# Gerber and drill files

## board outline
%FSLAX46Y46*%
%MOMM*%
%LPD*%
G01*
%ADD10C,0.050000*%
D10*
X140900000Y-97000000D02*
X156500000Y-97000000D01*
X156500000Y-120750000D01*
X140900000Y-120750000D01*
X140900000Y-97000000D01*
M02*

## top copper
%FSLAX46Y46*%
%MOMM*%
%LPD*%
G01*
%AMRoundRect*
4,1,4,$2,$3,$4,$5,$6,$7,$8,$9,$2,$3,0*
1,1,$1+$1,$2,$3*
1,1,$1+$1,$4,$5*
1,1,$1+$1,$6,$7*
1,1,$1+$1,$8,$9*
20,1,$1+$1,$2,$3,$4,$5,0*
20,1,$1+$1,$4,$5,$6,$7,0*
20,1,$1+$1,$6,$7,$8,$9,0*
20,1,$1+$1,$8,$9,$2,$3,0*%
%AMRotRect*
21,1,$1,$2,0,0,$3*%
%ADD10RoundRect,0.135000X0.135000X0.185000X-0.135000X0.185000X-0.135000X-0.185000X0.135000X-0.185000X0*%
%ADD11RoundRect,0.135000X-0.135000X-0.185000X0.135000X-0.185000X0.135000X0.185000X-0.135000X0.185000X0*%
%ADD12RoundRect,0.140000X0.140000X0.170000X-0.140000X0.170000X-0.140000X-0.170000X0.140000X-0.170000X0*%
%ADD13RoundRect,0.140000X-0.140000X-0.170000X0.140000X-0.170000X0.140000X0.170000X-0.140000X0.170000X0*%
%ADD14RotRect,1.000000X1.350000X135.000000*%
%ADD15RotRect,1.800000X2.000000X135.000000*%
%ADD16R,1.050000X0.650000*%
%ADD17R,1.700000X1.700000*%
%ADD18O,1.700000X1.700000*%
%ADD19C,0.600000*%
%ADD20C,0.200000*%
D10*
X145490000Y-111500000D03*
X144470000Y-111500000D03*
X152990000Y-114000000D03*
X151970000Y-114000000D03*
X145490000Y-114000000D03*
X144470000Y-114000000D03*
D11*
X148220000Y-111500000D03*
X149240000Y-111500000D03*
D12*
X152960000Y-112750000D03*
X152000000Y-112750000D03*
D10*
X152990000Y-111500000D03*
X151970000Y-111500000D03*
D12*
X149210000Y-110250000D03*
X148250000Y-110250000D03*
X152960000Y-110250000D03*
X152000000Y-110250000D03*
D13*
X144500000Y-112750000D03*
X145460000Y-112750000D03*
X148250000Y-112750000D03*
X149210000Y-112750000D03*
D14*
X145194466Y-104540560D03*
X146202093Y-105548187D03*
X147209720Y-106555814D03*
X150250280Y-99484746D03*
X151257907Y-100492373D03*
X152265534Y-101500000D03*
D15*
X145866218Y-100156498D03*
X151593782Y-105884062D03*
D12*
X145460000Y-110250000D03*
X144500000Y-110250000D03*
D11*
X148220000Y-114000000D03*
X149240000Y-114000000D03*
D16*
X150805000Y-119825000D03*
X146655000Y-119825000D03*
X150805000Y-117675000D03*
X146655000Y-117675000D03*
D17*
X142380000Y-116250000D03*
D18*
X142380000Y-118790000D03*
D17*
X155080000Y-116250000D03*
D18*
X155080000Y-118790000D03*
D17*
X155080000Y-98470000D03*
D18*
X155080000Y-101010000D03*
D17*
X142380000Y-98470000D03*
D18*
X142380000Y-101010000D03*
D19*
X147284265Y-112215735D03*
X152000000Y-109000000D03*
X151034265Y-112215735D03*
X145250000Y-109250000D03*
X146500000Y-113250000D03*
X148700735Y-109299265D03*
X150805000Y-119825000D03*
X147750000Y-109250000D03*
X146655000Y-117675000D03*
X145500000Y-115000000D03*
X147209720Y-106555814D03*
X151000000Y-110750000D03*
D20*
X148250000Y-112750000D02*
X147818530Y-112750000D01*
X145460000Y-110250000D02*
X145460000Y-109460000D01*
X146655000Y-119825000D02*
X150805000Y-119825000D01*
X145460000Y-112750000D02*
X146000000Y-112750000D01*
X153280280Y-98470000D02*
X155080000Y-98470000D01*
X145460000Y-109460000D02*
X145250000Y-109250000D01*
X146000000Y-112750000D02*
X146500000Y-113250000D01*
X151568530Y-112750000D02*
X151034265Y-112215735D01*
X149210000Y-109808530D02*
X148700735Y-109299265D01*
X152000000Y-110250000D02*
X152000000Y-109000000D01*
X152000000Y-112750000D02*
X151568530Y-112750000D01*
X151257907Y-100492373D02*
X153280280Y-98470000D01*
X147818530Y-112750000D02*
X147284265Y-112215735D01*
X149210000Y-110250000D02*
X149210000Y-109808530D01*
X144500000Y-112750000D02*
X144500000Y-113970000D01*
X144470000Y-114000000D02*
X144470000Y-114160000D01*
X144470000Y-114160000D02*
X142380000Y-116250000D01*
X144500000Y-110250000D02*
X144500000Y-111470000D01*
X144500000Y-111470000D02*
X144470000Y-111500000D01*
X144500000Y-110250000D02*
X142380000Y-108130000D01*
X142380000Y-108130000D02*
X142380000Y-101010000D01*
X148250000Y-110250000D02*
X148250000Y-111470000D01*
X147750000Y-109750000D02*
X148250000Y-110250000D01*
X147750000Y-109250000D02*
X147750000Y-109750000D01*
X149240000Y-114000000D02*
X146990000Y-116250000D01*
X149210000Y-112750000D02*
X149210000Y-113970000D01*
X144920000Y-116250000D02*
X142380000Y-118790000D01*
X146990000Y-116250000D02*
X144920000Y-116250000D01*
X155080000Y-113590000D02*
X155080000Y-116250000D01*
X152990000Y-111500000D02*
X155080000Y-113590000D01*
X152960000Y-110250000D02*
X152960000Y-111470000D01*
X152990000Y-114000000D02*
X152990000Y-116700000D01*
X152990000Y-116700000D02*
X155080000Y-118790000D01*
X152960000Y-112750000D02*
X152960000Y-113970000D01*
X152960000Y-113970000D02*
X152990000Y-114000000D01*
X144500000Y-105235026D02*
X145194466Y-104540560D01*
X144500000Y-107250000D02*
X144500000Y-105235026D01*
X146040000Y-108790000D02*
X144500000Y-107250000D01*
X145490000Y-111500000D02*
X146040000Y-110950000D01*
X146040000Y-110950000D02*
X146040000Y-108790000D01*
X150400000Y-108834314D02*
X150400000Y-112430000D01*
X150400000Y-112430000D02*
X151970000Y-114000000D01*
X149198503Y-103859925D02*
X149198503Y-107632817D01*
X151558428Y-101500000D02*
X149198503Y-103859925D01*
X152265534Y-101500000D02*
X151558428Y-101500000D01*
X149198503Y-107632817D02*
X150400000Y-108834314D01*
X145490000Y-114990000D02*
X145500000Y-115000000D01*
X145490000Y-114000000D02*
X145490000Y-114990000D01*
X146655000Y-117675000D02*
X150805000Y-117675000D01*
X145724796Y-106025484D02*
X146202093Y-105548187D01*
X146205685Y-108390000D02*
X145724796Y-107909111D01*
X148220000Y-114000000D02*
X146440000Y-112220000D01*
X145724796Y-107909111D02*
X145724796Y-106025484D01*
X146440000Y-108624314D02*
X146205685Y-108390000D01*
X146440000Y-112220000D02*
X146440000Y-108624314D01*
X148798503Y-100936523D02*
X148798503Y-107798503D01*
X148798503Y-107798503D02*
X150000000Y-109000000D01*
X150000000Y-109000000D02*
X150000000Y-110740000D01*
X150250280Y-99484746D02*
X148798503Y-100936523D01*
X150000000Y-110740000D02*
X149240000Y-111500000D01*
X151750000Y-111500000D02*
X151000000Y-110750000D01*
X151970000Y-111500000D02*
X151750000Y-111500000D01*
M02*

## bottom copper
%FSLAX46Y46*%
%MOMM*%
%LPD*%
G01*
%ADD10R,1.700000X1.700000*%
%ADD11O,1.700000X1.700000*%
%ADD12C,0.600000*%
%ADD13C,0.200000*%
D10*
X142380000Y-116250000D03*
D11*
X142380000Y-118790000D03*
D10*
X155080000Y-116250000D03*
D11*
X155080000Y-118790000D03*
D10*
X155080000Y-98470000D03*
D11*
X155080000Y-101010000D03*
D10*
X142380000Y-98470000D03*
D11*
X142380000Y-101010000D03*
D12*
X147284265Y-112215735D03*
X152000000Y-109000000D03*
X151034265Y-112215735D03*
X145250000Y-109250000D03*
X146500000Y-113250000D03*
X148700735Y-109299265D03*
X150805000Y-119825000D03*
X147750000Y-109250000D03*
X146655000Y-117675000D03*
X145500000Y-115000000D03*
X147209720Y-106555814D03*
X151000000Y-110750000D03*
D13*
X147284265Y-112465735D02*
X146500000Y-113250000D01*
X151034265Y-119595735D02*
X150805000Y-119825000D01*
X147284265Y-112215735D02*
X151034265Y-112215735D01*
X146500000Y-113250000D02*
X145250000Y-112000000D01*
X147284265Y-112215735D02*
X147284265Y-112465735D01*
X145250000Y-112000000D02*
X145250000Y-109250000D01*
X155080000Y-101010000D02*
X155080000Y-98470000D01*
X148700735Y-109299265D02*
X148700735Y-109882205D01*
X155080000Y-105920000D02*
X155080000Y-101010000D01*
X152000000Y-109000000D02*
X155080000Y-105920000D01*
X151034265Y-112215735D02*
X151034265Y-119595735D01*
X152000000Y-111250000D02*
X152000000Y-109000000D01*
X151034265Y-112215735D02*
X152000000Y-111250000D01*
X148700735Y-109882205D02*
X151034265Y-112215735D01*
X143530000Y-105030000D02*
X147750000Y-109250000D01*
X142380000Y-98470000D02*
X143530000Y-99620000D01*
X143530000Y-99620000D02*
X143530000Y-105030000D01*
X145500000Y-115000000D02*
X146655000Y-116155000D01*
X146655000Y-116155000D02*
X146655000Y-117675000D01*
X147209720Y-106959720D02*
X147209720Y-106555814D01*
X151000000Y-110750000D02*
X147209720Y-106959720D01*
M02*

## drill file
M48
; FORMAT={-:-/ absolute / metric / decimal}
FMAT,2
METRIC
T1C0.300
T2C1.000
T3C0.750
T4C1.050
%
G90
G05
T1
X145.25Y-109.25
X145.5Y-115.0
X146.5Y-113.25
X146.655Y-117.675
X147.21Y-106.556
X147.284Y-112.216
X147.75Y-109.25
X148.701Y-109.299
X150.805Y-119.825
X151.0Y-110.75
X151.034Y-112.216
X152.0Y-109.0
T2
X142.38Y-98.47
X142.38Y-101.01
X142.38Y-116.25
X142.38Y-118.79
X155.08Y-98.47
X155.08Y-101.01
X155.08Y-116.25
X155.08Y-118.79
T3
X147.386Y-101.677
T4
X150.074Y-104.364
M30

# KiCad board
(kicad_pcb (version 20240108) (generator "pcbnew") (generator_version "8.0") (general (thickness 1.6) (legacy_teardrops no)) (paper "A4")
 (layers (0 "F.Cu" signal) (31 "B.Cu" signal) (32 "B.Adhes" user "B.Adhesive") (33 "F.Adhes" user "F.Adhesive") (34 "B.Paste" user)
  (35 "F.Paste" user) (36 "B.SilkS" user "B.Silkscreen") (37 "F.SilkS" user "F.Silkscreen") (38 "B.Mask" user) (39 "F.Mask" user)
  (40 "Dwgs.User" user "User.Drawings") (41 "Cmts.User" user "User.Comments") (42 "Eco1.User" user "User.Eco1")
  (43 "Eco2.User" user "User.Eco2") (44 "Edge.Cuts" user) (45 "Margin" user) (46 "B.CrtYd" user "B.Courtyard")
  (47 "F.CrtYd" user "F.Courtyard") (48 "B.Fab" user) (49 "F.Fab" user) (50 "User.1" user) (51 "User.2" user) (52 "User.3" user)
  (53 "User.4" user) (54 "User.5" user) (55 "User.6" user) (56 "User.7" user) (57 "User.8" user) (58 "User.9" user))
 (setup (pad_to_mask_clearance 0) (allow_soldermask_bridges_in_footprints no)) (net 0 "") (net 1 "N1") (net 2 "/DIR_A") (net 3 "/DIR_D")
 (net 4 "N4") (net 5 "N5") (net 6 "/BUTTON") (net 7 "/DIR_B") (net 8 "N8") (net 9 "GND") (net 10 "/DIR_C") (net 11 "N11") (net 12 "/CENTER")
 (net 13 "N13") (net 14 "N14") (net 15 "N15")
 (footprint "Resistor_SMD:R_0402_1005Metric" (layer "F.Cu") (at 144.98 111.5 180)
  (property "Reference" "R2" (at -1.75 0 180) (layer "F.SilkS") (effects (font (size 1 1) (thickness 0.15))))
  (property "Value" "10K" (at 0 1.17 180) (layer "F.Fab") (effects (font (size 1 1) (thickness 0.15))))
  (pad "1" smd roundrect (at -0.51 0 180) (size 0.54 0.64) (layers "F.Cu" "F.Paste" "F.Mask") (roundrect_rratio 0.25) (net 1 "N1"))
  (pad "2" smd roundrect (at 0.51 0 180) (size 0.54 0.64) (layers "F.Cu" "F.Paste" "F.Mask") (roundrect_rratio 0.25) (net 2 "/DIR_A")))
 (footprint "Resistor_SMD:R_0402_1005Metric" (layer "F.Cu") (at 152.48 114 180)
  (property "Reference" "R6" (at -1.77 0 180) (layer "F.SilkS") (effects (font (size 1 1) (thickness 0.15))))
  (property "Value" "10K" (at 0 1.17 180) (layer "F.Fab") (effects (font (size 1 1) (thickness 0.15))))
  (pad "1" smd roundrect (at -0.51 0 180) (size 0.54 0.64) (layers "F.Cu" "F.Paste" "F.Mask") (roundrect_rratio 0.25) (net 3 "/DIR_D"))
  (pad "2" smd roundrect (at 0.51 0 180) (size 0.54 0.64) (layers "F.Cu" "F.Paste" "F.Mask") (roundrect_rratio 0.25) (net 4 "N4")))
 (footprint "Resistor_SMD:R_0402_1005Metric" (layer "F.Cu") (at 144.98 114 180)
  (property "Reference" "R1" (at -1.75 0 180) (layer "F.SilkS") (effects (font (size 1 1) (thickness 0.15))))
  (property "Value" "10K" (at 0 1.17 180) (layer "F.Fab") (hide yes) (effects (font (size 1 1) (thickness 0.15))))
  (pad "1" smd roundrect (at -0.51 0 180) (size 0.54 0.64) (layers "F.Cu" "F.Paste" "F.Mask") (roundrect_rratio 0.25) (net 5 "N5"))
  (pad "2" smd roundrect (at 0.51 0 180) (size 0.54 0.64) (layers "F.Cu" "F.Paste" "F.Mask") (roundrect_rratio 0.25) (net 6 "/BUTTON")))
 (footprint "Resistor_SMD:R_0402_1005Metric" (layer "F.Cu") (at 148.73 111.5)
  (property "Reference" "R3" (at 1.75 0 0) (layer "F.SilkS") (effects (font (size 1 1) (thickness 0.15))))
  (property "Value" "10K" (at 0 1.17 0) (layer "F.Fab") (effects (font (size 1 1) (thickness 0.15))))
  (pad "1" smd roundrect (at -0.51 0) (size 0.54 0.64) (layers "F.Cu" "F.Paste" "F.Mask") (roundrect_rratio 0.25) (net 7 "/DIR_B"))
  (pad "2" smd roundrect (at 0.51 0) (size 0.54 0.64) (layers "F.Cu" "F.Paste" "F.Mask") (roundrect_rratio 0.25) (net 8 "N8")))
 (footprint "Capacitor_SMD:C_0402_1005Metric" (layer "F.Cu") (at 152.48 112.75 180)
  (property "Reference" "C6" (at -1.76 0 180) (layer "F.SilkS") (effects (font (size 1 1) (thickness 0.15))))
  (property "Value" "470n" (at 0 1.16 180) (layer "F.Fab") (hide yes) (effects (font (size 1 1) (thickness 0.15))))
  (pad "1" smd roundrect (at -0.48 0 180) (size 0.56 0.62) (layers "F.Cu" "F.Paste" "F.Mask") (roundrect_rratio 0.25) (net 3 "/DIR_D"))
  (pad "2" smd roundrect (at 0.48 0 180) (size 0.56 0.62) (layers "F.Cu" "F.Paste" "F.Mask") (roundrect_rratio 0.25) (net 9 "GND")))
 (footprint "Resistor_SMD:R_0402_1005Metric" (layer "F.Cu") (at 152.48 111.5 180)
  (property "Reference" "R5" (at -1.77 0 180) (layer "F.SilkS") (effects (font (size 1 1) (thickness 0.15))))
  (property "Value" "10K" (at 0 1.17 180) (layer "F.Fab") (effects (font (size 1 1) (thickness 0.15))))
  (pad "1" smd roundrect (at -0.51 0 180) (size 0.54 0.64) (layers "F.Cu" "F.Paste" "F.Mask") (roundrect_rratio 0.25) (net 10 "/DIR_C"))
  (pad "2" smd roundrect (at 0.51 0 180) (size 0.54 0.64) (layers "F.Cu" "F.Paste" "F.Mask") (roundrect_rratio 0.25) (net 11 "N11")))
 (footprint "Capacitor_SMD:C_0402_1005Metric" (layer "F.Cu") (at 148.73 110.25 180)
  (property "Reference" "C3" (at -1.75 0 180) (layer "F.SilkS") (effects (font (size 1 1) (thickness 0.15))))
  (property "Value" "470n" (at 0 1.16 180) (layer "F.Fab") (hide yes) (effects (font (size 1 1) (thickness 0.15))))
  (pad "1" smd roundrect (at -0.48 0 180) (size 0.56 0.62) (layers "F.Cu" "F.Paste" "F.Mask") (roundrect_rratio 0.25) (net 9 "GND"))
  (pad "2" smd roundrect (at 0.48 0 180) (size 0.56 0.62) (layers "F.Cu" "F.Paste" "F.Mask") (roundrect_rratio 0.25) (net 7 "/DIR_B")))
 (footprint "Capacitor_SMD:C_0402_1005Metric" (layer "F.Cu") (at 152.48 110.25 180)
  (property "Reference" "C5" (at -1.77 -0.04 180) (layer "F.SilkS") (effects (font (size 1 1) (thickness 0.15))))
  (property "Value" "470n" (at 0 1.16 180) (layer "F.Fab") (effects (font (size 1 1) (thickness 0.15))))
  (pad "1" smd roundrect (at -0.48 0 180) (size 0.56 0.62) (layers "F.Cu" "F.Paste" "F.Mask") (roundrect_rratio 0.25) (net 10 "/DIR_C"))
  (pad "2" smd roundrect (at 0.48 0 180) (size 0.56 0.62) (layers "F.Cu" "F.Paste" "F.Mask") (roundrect_rratio 0.25) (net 9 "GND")))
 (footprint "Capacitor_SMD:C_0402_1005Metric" (layer "F.Cu") (at 144.98 112.75)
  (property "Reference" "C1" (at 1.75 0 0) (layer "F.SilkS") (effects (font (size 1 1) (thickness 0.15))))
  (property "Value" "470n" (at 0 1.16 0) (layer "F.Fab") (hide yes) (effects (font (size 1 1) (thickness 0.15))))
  (pad "1" smd roundrect (at -0.48 0) (size 0.56 0.62) (layers "F.Cu" "F.Paste" "F.Mask") (roundrect_rratio 0.25) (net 6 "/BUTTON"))
  (pad "2" smd roundrect (at 0.48 0) (size 0.56 0.62) (layers "F.Cu" "F.Paste" "F.Mask") (roundrect_rratio 0.25) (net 9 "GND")))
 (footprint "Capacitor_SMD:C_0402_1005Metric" (layer "F.Cu") (at 148.73 112.75)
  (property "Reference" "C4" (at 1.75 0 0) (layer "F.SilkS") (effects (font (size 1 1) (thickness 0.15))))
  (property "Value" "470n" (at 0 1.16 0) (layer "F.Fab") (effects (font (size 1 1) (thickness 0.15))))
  (pad "1" smd roundrect (at -0.48 0) (size 0.56 0.62) (layers "F.Cu" "F.Paste" "F.Mask") (roundrect_rratio 0.25) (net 9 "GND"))
  (pad "2" smd roundrect (at 0.48 0) (size 0.56 0.62) (layers "F.Cu" "F.Paste" "F.Mask") (roundrect_rratio 0.25) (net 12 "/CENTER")))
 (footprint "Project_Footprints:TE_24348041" (layer "F.Cu") (at 148.73 103.02028 45)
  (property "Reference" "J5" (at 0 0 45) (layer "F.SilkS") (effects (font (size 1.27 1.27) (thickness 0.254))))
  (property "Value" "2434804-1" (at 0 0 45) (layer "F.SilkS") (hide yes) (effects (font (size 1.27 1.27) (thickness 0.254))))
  (pad "" np_thru_hole circle (at 0 -1.9 45) (size 0.75 0.75) (drill 0.75) (layers "*.Cu" "*.Mask"))
  (pad "" np_thru_hole circle (at 0 1.9 45) (size 1.05 1.05) (drill 1.05) (layers "*.Cu" "*.Mask"))
  (pad "1" smd rect (at -3.575 -1.425 135) (size 1 1.35) (layers "F.Cu" "F.Paste" "F.Mask") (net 1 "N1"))
  (pad "2" smd rect (at -3.575 0 135) (size 1 1.35) (layers "F.Cu" "F.Paste" "F.Mask") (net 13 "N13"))
  (pad "3" smd rect (at -3.575 1.425 135) (size 1 1.35) (layers "F.Cu" "F.Paste" "F.Mask") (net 11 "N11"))
  (pad "4" smd rect (at 3.575 -1.425 135) (size 1 1.35) (layers "F.Cu" "F.Paste" "F.Mask") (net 8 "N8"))
  (pad "5" smd rect (at 3.575 0 135) (size 1 1.35) (layers "F.Cu" "F.Paste" "F.Mask") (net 9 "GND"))
  (pad "6" smd rect (at 3.575 1.425 135) (size 1 1.35) (layers "F.Cu" "F.Paste" "F.Mask") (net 4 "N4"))
  (pad "MP1" smd rect (at 0 -4.049999 135) (size 1.8 2) (layers "F.Cu" "F.Paste" "F.Mask") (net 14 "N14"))
  (pad "MP2" smd rect (at 0 4.049999 135) (size 1.8 2) (layers "F.Cu" "F.Paste" "F.Mask") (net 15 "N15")))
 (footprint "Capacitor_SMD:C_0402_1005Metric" (layer "F.Cu") (at 144.98 110.25 180)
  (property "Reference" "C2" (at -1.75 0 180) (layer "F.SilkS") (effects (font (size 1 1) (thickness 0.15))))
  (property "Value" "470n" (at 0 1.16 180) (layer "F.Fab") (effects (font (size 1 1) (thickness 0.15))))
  (pad "1" smd roundrect (at -0.48 0 180) (size 0.56 0.62) (layers "F.Cu" "F.Paste" "F.Mask") (roundrect_rratio 0.25) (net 9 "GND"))
  (pad "2" smd roundrect (at 0.48 0 180) (size 0.56 0.62) (layers "F.Cu" "F.Paste" "F.Mask") (roundrect_rratio 0.25) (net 2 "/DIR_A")))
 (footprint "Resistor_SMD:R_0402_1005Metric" (layer "F.Cu") (at 148.73 114)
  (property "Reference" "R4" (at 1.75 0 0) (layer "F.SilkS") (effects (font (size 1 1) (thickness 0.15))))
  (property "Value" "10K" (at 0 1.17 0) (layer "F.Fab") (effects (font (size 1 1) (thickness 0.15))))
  (pad "1" smd roundrect (at -0.51 0) (size 0.54 0.64) (layers "F.Cu" "F.Paste" "F.Mask") (roundrect_rratio 0.25) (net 13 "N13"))
  (pad "2" smd roundrect (at 0.51 0) (size 0.54 0.64) (layers "F.Cu" "F.Paste" "F.Mask") (roundrect_rratio 0.25) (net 12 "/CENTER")))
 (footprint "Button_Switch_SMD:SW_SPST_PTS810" (layer "F.Cu") (at 148.73 118.75 180)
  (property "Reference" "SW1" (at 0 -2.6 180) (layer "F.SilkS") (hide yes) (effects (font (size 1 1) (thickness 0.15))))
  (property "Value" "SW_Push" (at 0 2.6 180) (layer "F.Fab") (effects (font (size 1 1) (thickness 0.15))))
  (pad "1" smd rect (at -2.075 -1.075 180) (size 1.05 0.65) (layers "F.Cu" "F.Paste" "F.Mask") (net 9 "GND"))
  (pad "1" smd rect (at 2.075 -1.075 180) (size 1.05 0.65) (layers "F.Cu" "F.Paste" "F.Mask") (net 9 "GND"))
  (pad "2" smd rect (at -2.075 1.075 180) (size 1.05 0.65) (layers "F.Cu" "F.Paste" "F.Mask") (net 5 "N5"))
  (pad "2" smd rect (at 2.075 1.075 180) (size 1.05 0.65) (layers "F.Cu" "F.Paste" "F.Mask") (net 5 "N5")))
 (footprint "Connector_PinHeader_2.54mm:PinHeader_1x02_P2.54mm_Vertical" (layer "B.Cu") (at 142.38 116.25 180)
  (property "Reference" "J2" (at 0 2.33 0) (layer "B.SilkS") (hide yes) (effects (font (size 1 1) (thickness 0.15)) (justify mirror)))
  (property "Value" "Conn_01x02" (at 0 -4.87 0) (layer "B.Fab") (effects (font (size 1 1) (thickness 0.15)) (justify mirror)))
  (pad "1" thru_hole rect (at 0 0 180) (size 1.7 1.7) (drill 1) (layers "*.Cu" "*.Mask") (remove_unused_layers no) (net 6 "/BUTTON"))
  (pad "2" thru_hole oval (at 0 -2.54 180) (size 1.7 1.7) (drill 1) (layers "*.Cu" "*.Mask") (remove_unused_layers no) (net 12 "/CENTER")))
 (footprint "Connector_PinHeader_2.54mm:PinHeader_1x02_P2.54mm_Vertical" (layer "B.Cu") (at 155.08 116.25 180)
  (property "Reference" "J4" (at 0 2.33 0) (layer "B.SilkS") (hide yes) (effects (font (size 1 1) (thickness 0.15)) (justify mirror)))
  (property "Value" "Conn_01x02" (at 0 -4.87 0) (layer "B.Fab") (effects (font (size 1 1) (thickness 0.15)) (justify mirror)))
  (pad "1" thru_hole rect (at 0 0 180) (size 1.7 1.7) (drill 1) (layers "*.Cu" "*.Mask") (remove_unused_layers no) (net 10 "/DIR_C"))
  (pad "2" thru_hole oval (at 0 -2.54 180) (size 1.7 1.7) (drill 1) (layers "*.Cu" "*.Mask") (remove_unused_layers no) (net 3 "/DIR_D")))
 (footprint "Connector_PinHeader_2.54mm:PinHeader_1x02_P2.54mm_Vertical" (layer "B.Cu") (at 155.08 98.47 180)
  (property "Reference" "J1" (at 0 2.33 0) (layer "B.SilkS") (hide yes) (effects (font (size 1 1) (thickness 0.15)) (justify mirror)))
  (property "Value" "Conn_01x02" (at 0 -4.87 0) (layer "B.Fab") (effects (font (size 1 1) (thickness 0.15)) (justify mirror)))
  (pad "1" thru_hole rect (at 0 0 180) (size 1.7 1.7) (drill 1) (layers "*.Cu" "*.Mask") (remove_unused_layers no) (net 9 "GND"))
  (pad "2" thru_hole oval (at 0 -2.54 180) (size 1.7 1.7) (drill 1) (layers "*.Cu" "*.Mask") (remove_unused_layers no) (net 9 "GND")))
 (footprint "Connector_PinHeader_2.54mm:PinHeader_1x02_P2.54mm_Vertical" (layer "B.Cu") (at 142.38 98.47 180)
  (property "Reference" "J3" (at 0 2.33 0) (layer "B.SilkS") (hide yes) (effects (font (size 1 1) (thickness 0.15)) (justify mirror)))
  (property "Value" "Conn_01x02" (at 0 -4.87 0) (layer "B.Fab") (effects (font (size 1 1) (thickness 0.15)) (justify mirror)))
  (pad "1" thru_hole rect (at 0 0 180) (size 1.7 1.7) (drill 1) (layers "*.Cu" "*.Mask") (remove_unused_layers no) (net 7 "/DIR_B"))
  (pad "2" thru_hole oval (at 0 -2.54 180) (size 1.7 1.7) (drill 1) (layers "*.Cu" "*.Mask") (remove_unused_layers no) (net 2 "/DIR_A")))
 (gr_rect (start 140.9 97) (end 156.5 120.75) (stroke (width 0.05) (type default)) (fill none) (layer "Edge.Cuts"))
 (segment (start 148.25 112.75) (end 147.81853 112.75) (width 0.2) (layer "F.Cu") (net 9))
 (segment (start 145.46 110.25) (end 145.46 109.46) (width 0.2) (layer "F.Cu") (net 9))
 (segment (start 146.655 119.825) (end 150.805 119.825) (width 0.2) (layer "F.Cu") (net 9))
 (segment (start 145.46 112.75) (end 146 112.75) (width 0.2) (layer "F.Cu") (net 9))
 (segment (start 153.28028 98.47) (end 155.08 98.47) (width 0.2) (layer "F.Cu") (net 9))
 (segment (start 145.46 109.46) (end 145.25 109.25) (width 0.2) (layer "F.Cu") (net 9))
 (segment (start 146 112.75) (end 146.5 113.25) (width 0.2) (layer "F.Cu") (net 9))
 (segment (start 151.56853 112.75) (end 151.034265 112.215735) (width 0.2) (layer "F.Cu") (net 9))
 (segment (start 149.21 109.80853) (end 148.700735 109.299265) (width 0.2) (layer "F.Cu") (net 9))
 (segment (start 152 110.25) (end 152 109) (width 0.2) (layer "F.Cu") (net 9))
 (segment (start 152 112.75) (end 151.56853 112.75) (width 0.2) (layer "F.Cu") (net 9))
 (segment (start 151.257907 100.492373) (end 153.28028 98.47) (width 0.2) (layer "F.Cu") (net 9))
 (segment (start 147.81853 112.75) (end 147.284265 112.215735) (width 0.2) (layer "F.Cu") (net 9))
 (segment (start 149.21 110.25) (end 149.21 109.80853) (width 0.2) (layer "F.Cu") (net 9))
 (via (at 147.284265 112.215735) (size 0.6) (drill 0.3) (layers "F.Cu" "B.Cu") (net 9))
 (via (at 152 109) (size 0.6) (drill 0.3) (layers "F.Cu" "B.Cu") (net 9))
 (via (at 151.034265 112.215735) (size 0.6) (drill 0.3) (layers "F.Cu" "B.Cu") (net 9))
 (via (at 145.25 109.25) (size 0.6) (drill 0.3) (layers "F.Cu" "B.Cu") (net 9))
 (via (at 146.5 113.25) (size 0.6) (drill 0.3) (layers "F.Cu" "B.Cu") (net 9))
 (via (at 148.700735 109.299265) (size 0.6) (drill 0.3) (layers "F.Cu" "B.Cu") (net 9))
 (via (at 150.805 119.825) (size 0.6) (drill 0.3) (layers "F.Cu" "B.Cu") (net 9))
 (segment (start 147.284265 112.465735) (end 146.5 113.25) (width 0.2) (layer "B.Cu") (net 9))
 (segment (start 151.034265 119.595735) (end 150.805 119.825) (width 0.2) (layer "B.Cu") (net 9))
 (segment (start 147.284265 112.215735) (end 151.034265 112.215735) (width 0.2) (layer "B.Cu") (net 9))
 (segment (start 146.5 113.25) (end 145.25 112) (width 0.2) (layer "B.Cu") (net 9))
 (segment (start 147.284265 112.215735) (end 147.284265 112.465735) (width 0.2) (layer "B.Cu") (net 9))
 (segment (start 145.25 112) (end 145.25 109.25) (width 0.2) (layer "B.Cu") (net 9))
 (segment (start 155.08 101.01) (end 155.08 98.47) (width 0.2) (layer "B.Cu") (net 9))
 (segment (start 148.700735 109.299265) (end 148.700735 109.882205) (width 0.2) (layer "B.Cu") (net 9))
 (segment (start 155.08 105.92) (end 155.08 101.01) (width 0.2) (layer "B.Cu") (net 9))
 (segment (start 152 109) (end 155.08 105.92) (width 0.2) (layer "B.Cu") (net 9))
 (segment (start 151.034265 112.215735) (end 151.034265 119.595735) (width 0.2) (layer "B.Cu") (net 9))
 (segment (start 152 111.25) (end 152 109) (width 0.2) (layer "B.Cu") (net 9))
 (segment (start 151.034265 112.215735) (end 152 111.25) (width 0.2) (layer "B.Cu") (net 9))
 (segment (start 148.700735 109.882205) (end 151.034265 112.215735) (width 0.2) (layer "B.Cu") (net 9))
 (segment (start 144.5 112.75) (end 144.5 113.97) (width 0.2) (layer "F.Cu") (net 6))
 (segment (start 144.47 114) (end 144.47 114.16) (width 0.2) (layer "F.Cu") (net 6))
 (segment (start 144.47 114.16) (end 142.38 116.25) (width 0.2) (layer "F.Cu") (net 6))
 (segment (start 144.5 110.25) (end 144.5 111.47) (width 0.2) (layer "F.Cu") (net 2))
 (segment (start 144.5 111.47) (end 144.47 111.5) (width 0.2) (layer "F.Cu") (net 2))
 (segment (start 144.5 110.25) (end 142.38 108.13) (width 0.2) (layer "F.Cu") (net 2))
 (segment (start 142.38 108.13) (end 142.38 101.01) (width 0.2) (layer "F.Cu") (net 2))
 (segment (start 148.25 110.25) (end 148.25 111.47) (width 0.2) (layer "F.Cu") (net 7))
 (segment (start 147.75 109.75) (end 148.25 110.25) (width 0.2) (layer "F.Cu") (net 7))
 (segment (start 147.75 109.25) (end 147.75 109.75) (width 0.2) (layer "F.Cu") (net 7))
 (via (at 147.75 109.25) (size 0.6) (drill 0.3) (layers "F.Cu" "B.Cu") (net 7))
 (segment (start 143.53 105.03) (end 147.75 109.25) (width 0.2) (layer "B.Cu") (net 7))
 (segment (start 142.38 98.47) (end 143.53 99.62) (width 0.2) (layer "B.Cu") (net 7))
 (segment (start 143.53 99.62) (end 143.53 105.03) (width 0.2) (layer "B.Cu") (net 7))
 (segment (start 149.24 114) (end 146.99 116.25) (width 0.2) (layer "F.Cu") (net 12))
 (segment (start 149.21 112.75) (end 149.21 113.97) (width 0.2) (layer "F.Cu") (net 12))
 (segment (start 144.92 116.25) (end 142.38 118.79) (width 0.2) (layer "F.Cu") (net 12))
 (segment (start 146.99 116.25) (end 144.92 116.25) (width 0.2) (layer "F.Cu") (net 12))
 (segment (start 155.08 113.59) (end 155.08 116.25) (width 0.2) (layer "F.Cu") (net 10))
 (segment (start 152.99 111.5) (end 155.08 113.59) (width 0.2) (layer "F.Cu") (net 10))
 (segment (start 152.96 110.25) (end 152.96 111.47) (width 0.2) (layer "F.Cu") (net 10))
 (segment (start 152.99 114) (end 152.99 116.7) (width 0.2) (layer "F.Cu") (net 3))
 (segment (start 152.99 116.7) (end 155.08 118.79) (width 0.2) (layer "F.Cu") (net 3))
 (segment (start 152.96 112.75) (end 152.96 113.97) (width 0.2) (layer "F.Cu") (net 3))
 (segment (start 152.96 113.97) (end 152.99 114) (width 0.2) (layer "F.Cu") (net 3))
 (segment (start 144.5 105.235026) (end 145.194466 104.54056) (width 0.2) (layer "F.Cu") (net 1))
 (segment (start 144.5 107.25) (end 144.5 105.235026) (width 0.2) (layer "F.Cu") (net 1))
 (segment (start 146.04 108.79) (end 144.5 107.25) (width 0.2) (layer "F.Cu") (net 1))
 (segment (start 145.49 111.5) (end 146.04 110.95) (width 0.2) (layer "F.Cu") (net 1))
 (segment (start 146.04 110.95) (end 146.04 108.79) (width 0.2) (layer "F.Cu") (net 1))
 (segment (start 150.4 108.834314) (end 150.4 112.43) (width 0.2) (layer "F.Cu") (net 4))
 (segment (start 150.4 112.43) (end 151.97 114) (width 0.2) (layer "F.Cu") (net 4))
 (segment (start 149.198503 103.859925) (end 149.198503 107.632817) (width 0.2) (layer "F.Cu") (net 4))
 (segment (start 151.558428 101.5) (end 149.198503 103.859925) (width 0.2) (layer "F.Cu") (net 4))
 (segment (start 152.265534 101.5) (end 151.558428 101.5) (width 0.2) (layer "F.Cu") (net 4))
 (segment (start 149.198503 107.632817) (end 150.4 108.834314) (width 0.2) (layer "F.Cu") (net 4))
 (segment (start 145.49 114.99) (end 145.5 115) (width 0.2) (layer "F.Cu") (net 5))
 (segment (start 145.49 114) (end 145.49 114.99) (width 0.2) (layer "F.Cu") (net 5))
 (segment (start 146.655 117.675) (end 150.805 117.675) (width 0.2) (layer "F.Cu") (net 5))
 (via (at 146.655 117.675) (size 0.6) (drill 0.3) (layers "F.Cu" "B.Cu") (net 5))
 (via (at 145.5 115) (size 0.6) (drill 0.3) (layers "F.Cu" "B.Cu") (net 5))
 (segment (start 145.5 115) (end 146.655 116.155) (width 0.2) (layer "B.Cu") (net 5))
 (segment (start 146.655 116.155) (end 146.655 117.675) (width 0.2) (layer "B.Cu") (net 5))
 (segment (start 145.724796 106.025484) (end 146.202093 105.548187) (width 0.2) (layer "F.Cu") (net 13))
 (segment (start 146.205685 108.39) (end 145.724796 107.909111) (width 0.2) (layer "F.Cu") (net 13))
 (segment (start 148.22 114) (end 146.44 112.22) (width 0.2) (layer "F.Cu") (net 13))
 (segment (start 145.724796 107.909111) (end 145.724796 106.025484) (width 0.2) (layer "F.Cu") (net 13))
 (segment (start 146.44 108.624314) (end 146.205685 108.39) (width 0.2) (layer "F.Cu") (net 13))
 (segment (start 146.44 112.22) (end 146.44 108.624314) (width 0.2) (layer "F.Cu") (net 13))
 (segment (start 148.798503 100.936523) (end 148.798503 107.798503) (width 0.2) (layer "F.Cu") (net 8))
 (segment (start 148.798503 107.798503) (end 150 109) (width 0.2) (layer "F.Cu") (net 8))
 (segment (start 150 109) (end 150 110.74) (width 0.2) (layer "F.Cu") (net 8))
 (segment (start 150.25028 99.484746) (end 148.798503 100.936523) (width 0.2) (layer "F.Cu") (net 8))
 (segment (start 150 110.74) (end 149.24 111.5) (width 0.2) (layer "F.Cu") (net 8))
 (segment (start 151.75 111.5) (end 151 110.75) (width 0.2) (layer "F.Cu") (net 11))
 (segment (start 151.97 111.5) (end 151.75 111.5) (width 0.2) (layer "F.Cu") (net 11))
 (via (at 147.20972 106.555814) (size 0.6) (drill 0.3) (layers "F.Cu" "B.Cu") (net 11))
 (via (at 151 110.75) (size 0.6) (drill 0.3) (layers "F.Cu" "B.Cu") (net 11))
 (segment (start 147.20972 106.95972) (end 147.20972 106.555814) (width 0.2) (layer "B.Cu") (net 11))
 (segment (start 151 110.75) (end 147.20972 106.95972) (width 0.2) (layer "B.Cu") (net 11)))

